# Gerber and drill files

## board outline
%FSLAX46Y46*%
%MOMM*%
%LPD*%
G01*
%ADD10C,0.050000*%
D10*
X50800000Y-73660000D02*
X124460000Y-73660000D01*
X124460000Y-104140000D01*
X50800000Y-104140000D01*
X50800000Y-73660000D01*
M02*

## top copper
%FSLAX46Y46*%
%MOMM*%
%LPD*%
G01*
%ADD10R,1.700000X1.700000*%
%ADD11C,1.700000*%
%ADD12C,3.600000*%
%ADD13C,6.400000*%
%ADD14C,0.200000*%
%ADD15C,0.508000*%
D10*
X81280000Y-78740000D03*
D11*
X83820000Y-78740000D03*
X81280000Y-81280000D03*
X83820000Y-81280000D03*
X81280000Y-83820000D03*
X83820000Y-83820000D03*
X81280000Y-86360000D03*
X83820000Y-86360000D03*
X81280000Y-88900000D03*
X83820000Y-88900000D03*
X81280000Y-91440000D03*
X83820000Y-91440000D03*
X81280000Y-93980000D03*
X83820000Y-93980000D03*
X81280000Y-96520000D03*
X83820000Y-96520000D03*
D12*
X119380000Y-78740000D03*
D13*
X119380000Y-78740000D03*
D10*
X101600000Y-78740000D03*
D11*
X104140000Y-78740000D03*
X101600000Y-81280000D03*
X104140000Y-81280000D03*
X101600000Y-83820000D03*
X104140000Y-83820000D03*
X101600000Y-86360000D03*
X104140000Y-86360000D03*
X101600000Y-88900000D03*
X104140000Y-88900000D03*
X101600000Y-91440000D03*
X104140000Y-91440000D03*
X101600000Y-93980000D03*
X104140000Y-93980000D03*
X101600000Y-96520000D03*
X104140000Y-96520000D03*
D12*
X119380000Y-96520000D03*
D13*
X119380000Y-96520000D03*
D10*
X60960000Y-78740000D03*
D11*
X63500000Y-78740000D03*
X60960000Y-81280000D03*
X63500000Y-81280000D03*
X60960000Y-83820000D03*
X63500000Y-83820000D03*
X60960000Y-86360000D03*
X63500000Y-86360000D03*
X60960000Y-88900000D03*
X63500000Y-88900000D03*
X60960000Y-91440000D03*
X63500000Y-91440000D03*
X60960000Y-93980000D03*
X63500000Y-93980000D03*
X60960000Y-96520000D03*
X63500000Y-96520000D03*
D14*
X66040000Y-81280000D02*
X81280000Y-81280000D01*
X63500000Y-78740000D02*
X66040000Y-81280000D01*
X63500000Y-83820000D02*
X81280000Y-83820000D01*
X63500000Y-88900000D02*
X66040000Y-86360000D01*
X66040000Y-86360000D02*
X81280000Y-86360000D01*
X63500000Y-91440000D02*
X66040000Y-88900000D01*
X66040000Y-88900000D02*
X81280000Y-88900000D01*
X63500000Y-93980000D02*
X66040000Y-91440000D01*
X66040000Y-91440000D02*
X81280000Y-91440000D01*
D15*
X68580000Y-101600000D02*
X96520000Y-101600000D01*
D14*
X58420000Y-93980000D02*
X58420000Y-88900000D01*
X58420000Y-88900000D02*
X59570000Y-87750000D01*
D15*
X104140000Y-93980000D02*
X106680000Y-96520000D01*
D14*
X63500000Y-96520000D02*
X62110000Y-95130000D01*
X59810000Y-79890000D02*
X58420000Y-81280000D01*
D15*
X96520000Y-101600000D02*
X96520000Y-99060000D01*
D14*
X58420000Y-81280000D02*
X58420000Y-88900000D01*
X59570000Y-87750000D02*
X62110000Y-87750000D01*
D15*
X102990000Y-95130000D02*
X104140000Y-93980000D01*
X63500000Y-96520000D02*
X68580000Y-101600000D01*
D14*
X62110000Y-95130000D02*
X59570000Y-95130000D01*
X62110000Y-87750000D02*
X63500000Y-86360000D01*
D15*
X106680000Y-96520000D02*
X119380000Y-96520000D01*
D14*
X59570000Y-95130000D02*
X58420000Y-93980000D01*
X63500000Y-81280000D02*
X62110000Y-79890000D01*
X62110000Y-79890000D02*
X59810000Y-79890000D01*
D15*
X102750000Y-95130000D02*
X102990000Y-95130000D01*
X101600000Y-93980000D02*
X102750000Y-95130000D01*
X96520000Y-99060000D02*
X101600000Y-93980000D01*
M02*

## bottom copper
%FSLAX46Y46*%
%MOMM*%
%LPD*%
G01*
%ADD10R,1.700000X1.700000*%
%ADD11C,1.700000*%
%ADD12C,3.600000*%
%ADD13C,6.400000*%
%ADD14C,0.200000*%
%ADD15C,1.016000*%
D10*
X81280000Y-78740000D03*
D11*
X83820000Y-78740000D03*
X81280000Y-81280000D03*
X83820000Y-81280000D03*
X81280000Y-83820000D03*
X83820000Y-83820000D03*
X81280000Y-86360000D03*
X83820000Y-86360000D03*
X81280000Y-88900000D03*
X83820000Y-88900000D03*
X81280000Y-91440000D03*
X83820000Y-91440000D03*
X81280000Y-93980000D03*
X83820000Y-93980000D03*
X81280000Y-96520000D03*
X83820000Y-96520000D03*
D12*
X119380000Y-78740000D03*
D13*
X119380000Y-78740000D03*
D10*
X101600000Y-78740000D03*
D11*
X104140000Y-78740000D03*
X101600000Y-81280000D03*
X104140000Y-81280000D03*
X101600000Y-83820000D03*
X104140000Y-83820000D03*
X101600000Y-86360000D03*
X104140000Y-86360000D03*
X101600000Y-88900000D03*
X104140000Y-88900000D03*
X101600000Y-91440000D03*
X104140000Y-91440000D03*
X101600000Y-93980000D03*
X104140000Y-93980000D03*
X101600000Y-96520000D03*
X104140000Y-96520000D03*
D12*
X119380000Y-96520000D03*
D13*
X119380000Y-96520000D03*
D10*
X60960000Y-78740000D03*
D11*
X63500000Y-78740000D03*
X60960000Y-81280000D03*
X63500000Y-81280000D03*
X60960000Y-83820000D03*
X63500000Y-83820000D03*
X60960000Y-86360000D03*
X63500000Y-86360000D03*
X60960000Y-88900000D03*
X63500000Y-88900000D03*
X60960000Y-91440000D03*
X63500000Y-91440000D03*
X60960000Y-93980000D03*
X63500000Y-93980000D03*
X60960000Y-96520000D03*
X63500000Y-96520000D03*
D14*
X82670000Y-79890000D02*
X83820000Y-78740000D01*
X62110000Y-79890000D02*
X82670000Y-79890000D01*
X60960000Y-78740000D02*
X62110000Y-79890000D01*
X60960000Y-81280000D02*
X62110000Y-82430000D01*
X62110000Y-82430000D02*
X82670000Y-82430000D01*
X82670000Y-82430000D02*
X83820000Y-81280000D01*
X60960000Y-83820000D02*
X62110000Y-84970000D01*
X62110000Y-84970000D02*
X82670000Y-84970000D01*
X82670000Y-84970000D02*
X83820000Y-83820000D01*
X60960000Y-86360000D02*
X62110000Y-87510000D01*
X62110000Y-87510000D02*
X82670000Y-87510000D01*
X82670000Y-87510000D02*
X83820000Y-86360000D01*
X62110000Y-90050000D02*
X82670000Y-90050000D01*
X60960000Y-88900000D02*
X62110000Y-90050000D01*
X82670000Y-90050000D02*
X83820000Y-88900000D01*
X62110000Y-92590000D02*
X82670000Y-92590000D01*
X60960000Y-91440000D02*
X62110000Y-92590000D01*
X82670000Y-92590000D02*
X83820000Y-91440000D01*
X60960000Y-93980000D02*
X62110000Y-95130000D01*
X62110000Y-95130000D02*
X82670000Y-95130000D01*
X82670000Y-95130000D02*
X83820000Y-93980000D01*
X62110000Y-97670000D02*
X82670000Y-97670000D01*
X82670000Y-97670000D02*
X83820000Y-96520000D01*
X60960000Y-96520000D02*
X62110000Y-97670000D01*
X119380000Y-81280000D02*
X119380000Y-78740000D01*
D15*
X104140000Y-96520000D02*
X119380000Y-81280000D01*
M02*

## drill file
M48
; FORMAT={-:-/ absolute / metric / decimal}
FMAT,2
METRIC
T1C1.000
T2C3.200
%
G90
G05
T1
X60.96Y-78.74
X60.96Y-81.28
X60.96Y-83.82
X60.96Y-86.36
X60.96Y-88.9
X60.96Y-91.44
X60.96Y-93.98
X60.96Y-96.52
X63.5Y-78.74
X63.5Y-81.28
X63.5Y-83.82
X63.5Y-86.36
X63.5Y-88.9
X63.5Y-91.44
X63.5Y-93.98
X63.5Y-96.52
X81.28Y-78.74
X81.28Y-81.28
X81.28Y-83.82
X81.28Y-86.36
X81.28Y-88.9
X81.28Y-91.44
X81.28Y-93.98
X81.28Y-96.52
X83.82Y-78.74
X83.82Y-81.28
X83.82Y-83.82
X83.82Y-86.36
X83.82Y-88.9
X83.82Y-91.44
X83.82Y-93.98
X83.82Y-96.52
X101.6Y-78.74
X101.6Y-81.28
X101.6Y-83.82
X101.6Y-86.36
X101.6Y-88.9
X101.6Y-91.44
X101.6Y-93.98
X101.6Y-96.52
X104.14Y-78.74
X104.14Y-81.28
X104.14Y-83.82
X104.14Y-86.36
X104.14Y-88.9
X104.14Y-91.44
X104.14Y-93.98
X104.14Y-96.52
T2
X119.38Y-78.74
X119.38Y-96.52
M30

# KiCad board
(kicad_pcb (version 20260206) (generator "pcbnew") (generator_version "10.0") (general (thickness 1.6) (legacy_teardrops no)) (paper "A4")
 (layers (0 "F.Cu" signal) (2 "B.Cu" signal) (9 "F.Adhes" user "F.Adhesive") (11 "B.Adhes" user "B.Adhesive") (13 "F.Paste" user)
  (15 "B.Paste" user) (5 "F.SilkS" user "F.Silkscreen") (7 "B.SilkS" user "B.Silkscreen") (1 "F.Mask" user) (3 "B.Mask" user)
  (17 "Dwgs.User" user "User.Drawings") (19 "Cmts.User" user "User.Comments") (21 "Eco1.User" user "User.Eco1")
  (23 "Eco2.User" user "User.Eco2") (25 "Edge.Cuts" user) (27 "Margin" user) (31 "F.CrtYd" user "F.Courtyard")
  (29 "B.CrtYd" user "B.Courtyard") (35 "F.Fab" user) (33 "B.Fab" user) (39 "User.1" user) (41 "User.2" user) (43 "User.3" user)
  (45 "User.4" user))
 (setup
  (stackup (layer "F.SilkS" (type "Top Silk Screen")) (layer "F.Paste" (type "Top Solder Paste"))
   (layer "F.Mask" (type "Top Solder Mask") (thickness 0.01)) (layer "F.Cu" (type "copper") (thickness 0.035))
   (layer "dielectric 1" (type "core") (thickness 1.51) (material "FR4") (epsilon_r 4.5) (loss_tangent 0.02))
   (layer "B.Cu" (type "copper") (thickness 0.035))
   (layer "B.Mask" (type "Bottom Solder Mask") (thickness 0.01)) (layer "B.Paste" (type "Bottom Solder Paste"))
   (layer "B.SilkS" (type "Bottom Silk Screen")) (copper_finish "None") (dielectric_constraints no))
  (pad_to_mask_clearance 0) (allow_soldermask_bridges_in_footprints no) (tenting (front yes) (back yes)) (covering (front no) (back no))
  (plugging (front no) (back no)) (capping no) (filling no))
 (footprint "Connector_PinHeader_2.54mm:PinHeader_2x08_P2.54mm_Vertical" (layer "F.Cu") (at 81.28 78.74)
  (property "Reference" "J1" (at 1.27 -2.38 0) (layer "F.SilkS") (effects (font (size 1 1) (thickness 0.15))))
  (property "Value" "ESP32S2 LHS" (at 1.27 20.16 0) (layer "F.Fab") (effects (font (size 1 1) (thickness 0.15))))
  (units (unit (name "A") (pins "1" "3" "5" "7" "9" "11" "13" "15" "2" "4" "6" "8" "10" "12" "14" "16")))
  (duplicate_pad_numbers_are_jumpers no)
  (pad "1" thru_hole rect (at 0 0) (size 1.7 1.7) (drill 1) (layers "*.Cu" "*.Mask") (remove_unused_layers no)
   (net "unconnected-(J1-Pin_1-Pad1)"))
  (pad "2" thru_hole circle (at 2.54 0) (size 1.7 1.7) (drill 1) (layers "*.Cu" "*.Mask") (remove_unused_layers no) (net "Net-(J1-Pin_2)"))
  (pad "3" thru_hole circle (at 0 2.54) (size 1.7 1.7) (drill 1) (layers "*.Cu" "*.Mask") (remove_unused_layers no) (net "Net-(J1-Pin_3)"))
  (pad "4" thru_hole circle (at 2.54 2.54) (size 1.7 1.7) (drill 1) (layers "*.Cu" "*.Mask") (remove_unused_layers no)
   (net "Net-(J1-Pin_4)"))
  (pad "5" thru_hole circle (at 0 5.08) (size 1.7 1.7) (drill 1) (layers "*.Cu" "*.Mask") (remove_unused_layers no) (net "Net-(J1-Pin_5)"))
  (pad "6" thru_hole circle (at 2.54 5.08) (size 1.7 1.7) (drill 1) (layers "*.Cu" "*.Mask") (remove_unused_layers no)
   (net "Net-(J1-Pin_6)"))
  (pad "7" thru_hole circle (at 0 7.62) (size 1.7 1.7) (drill 1) (layers "*.Cu" "*.Mask") (remove_unused_layers no) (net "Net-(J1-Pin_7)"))
  (pad "8" thru_hole circle (at 2.54 7.62) (size 1.7 1.7) (drill 1) (layers "*.Cu" "*.Mask") (remove_unused_layers no)
   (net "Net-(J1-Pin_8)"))
  (pad "9" thru_hole circle (at 0 10.16) (size 1.7 1.7) (drill 1) (layers "*.Cu" "*.Mask") (remove_unused_layers no) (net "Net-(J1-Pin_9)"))
  (pad "10" thru_hole circle (at 2.54 10.16) (size 1.7 1.7) (drill 1) (layers "*.Cu" "*.Mask") (remove_unused_layers no)
   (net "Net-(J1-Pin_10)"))
  (pad "11" thru_hole circle (at 0 12.7) (size 1.7 1.7) (drill 1) (layers "*.Cu" "*.Mask") (remove_unused_layers no) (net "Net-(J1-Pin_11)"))
  (pad "12" thru_hole circle (at 2.54 12.7) (size 1.7 1.7) (drill 1) (layers "*.Cu" "*.Mask") (remove_unused_layers no)
   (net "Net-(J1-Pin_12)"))
  (pad "13" thru_hole circle (at 0 15.24) (size 1.7 1.7) (drill 1) (layers "*.Cu" "*.Mask") (remove_unused_layers no)
   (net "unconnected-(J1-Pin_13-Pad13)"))
  (pad "14" thru_hole circle (at 2.54 15.24) (size 1.7 1.7) (drill 1) (layers "*.Cu" "*.Mask") (remove_unused_layers no)
   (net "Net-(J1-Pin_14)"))
  (pad "15" thru_hole circle (at 0 17.78) (size 1.7 1.7) (drill 1) (layers "*.Cu" "*.Mask") (remove_unused_layers no)
   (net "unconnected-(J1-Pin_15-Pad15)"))
  (pad "16" thru_hole circle (at 2.54 17.78) (size 1.7 1.7) (drill 1) (layers "*.Cu" "*.Mask") (remove_unused_layers no)
   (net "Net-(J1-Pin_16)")))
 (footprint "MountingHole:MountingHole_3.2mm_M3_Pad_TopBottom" (layer "F.Cu") (at 119.38 78.74)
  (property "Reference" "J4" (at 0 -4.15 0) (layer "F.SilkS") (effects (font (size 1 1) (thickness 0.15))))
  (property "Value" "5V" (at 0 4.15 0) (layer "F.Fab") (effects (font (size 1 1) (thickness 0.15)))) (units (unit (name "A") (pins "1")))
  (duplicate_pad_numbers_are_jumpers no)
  (pad "1" thru_hole circle (at 0 0) (size 3.6 3.6) (drill 3.2) (layers "*.Cu" "*.Mask") (remove_unused_layers no) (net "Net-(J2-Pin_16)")
   (zone_connect 2))
  (pad "1" connect circle (at 0 0) (size 6.4 6.4) (layers "F.Cu" "F.Mask") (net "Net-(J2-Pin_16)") (zone_connect 2))
  (pad "1" connect circle (at 0 0) (size 6.4 6.4) (layers "B.Cu" "B.Mask") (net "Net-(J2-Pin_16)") (zone_connect 2)))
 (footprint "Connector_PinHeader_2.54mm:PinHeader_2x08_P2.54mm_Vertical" (layer "F.Cu") (at 101.6 78.74)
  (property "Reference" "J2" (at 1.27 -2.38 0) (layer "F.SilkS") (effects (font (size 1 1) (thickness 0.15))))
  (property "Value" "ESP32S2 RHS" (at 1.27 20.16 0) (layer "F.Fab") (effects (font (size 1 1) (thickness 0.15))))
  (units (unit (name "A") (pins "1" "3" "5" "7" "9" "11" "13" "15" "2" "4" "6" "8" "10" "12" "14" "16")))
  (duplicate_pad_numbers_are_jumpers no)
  (pad "1" thru_hole rect (at 0 0) (size 1.7 1.7) (drill 1) (layers "*.Cu" "*.Mask") (remove_unused_layers no)
   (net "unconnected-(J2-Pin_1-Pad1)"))
  (pad "2" thru_hole circle (at 2.54 0) (size 1.7 1.7) (drill 1) (layers "*.Cu" "*.Mask") (remove_unused_layers no)
   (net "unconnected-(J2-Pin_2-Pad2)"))
  (pad "3" thru_hole circle (at 0 2.54) (size 1.7 1.7) (drill 1) (layers "*.Cu" "*.Mask") (remove_unused_layers no)
   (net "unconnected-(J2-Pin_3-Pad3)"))
  (pad "4" thru_hole circle (at 2.54 2.54) (size 1.7 1.7) (drill 1) (layers "*.Cu" "*.Mask") (remove_unused_layers no)
   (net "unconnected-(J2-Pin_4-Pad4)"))
  (pad "5" thru_hole circle (at 0 5.08) (size 1.7 1.7) (drill 1) (layers "*.Cu" "*.Mask") (remove_unused_layers no)
   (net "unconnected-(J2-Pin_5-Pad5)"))
  (pad "6" thru_hole circle (at 2.54 5.08) (size 1.7 1.7) (drill 1) (layers "*.Cu" "*.Mask") (remove_unused_layers no)
   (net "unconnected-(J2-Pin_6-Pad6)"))
  (pad "7" thru_hole circle (at 0 7.62) (size 1.7 1.7) (drill 1) (layers "*.Cu" "*.Mask") (remove_unused_layers no)
   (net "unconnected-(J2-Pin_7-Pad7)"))
  (pad "8" thru_hole circle (at 2.54 7.62) (size 1.7 1.7) (drill 1) (layers "*.Cu" "*.Mask") (remove_unused_layers no)
   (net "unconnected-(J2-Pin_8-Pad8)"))
  (pad "9" thru_hole circle (at 0 10.16) (size 1.7 1.7) (drill 1) (layers "*.Cu" "*.Mask") (remove_unused_layers no)
   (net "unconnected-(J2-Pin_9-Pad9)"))
  (pad "10" thru_hole circle (at 2.54 10.16) (size 1.7 1.7) (drill 1) (layers "*.Cu" "*.Mask") (remove_unused_layers no)
   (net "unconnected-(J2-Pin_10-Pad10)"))
  (pad "11" thru_hole circle (at 0 12.7) (size 1.7 1.7) (drill 1) (layers "*.Cu" "*.Mask") (remove_unused_layers no)
   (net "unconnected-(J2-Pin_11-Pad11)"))
  (pad "12" thru_hole circle (at 2.54 12.7) (size 1.7 1.7) (drill 1) (layers "*.Cu" "*.Mask") (remove_unused_layers no)
   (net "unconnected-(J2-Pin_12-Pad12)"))
  (pad "13" thru_hole circle (at 0 15.24) (size 1.7 1.7) (drill 1) (layers "*.Cu" "*.Mask") (remove_unused_layers no)
   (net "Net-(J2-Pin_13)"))
  (pad "14" thru_hole circle (at 2.54 15.24) (size 1.7 1.7) (drill 1) (layers "*.Cu" "*.Mask") (remove_unused_layers no)
   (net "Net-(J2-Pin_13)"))
  (pad "15" thru_hole circle (at 0 17.78) (size 1.7 1.7) (drill 1) (layers "*.Cu" "*.Mask") (remove_unused_layers no)
   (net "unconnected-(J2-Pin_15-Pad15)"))
  (pad "16" thru_hole circle (at 2.54 17.78) (size 1.7 1.7) (drill 1) (layers "*.Cu" "*.Mask") (remove_unused_layers no)
   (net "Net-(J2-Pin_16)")))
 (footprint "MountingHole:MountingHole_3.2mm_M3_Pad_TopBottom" (layer "F.Cu") (at 119.38 96.52)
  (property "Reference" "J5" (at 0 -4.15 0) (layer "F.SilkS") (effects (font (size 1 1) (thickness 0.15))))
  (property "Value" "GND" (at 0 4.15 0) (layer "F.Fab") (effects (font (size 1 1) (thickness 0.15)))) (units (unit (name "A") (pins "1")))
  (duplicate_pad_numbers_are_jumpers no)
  (pad "1" thru_hole circle (at 0 0) (size 3.6 3.6) (drill 3.2) (layers "*.Cu" "*.Mask") (remove_unused_layers no) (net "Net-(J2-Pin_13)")
   (zone_connect 2))
  (pad "1" connect circle (at 0 0) (size 6.4 6.4) (layers "F.Cu" "F.Mask") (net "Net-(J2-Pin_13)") (zone_connect 2))
  (pad "1" connect circle (at 0 0) (size 6.4 6.4) (layers "B.Cu" "B.Mask") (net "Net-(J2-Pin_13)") (zone_connect 2)))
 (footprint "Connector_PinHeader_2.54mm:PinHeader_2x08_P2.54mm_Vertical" (layer "F.Cu") (at 60.96 78.74)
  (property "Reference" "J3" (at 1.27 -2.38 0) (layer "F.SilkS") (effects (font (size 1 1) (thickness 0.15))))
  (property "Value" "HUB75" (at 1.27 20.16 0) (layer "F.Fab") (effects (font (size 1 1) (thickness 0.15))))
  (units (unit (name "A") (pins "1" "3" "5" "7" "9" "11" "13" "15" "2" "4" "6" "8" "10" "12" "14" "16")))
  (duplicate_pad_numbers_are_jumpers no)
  (pad "1" thru_hole rect (at 0 0) (size 1.7 1.7) (drill 1) (layers "*.Cu" "*.Mask") (remove_unused_layers no) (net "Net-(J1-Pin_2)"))
  (pad "2" thru_hole circle (at 2.54 0) (size 1.7 1.7) (drill 1) (layers "*.Cu" "*.Mask") (remove_unused_layers no) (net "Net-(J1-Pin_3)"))
  (pad "3" thru_hole circle (at 0 2.54) (size 1.7 1.7) (drill 1) (layers "*.Cu" "*.Mask") (remove_unused_layers no) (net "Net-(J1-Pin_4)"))
  (pad "4" thru_hole circle (at 2.54 2.54) (size 1.7 1.7) (drill 1) (layers "*.Cu" "*.Mask") (remove_unused_layers no)
   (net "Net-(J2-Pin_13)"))
  (pad "5" thru_hole circle (at 0 5.08) (size 1.7 1.7) (drill 1) (layers "*.Cu" "*.Mask") (remove_unused_layers no) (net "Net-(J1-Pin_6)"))
  (pad "6" thru_hole circle (at 2.54 5.08) (size 1.7 1.7) (drill 1) (layers "*.Cu" "*.Mask") (remove_unused_layers no)
   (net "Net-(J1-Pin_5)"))
  (pad "7" thru_hole circle (at 0 7.62) (size 1.7 1.7) (drill 1) (layers "*.Cu" "*.Mask") (remove_unused_layers no) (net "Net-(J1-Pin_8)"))
  (pad "8" thru_hole circle (at 2.54 7.62) (size 1.7 1.7) (drill 1) (layers "*.Cu" "*.Mask") (remove_unused_layers no)
   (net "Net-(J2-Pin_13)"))
  (pad "9" thru_hole circle (at 0 10.16) (size 1.7 1.7) (drill 1) (layers "*.Cu" "*.Mask") (remove_unused_layers no) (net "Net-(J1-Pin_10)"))
  (pad "10" thru_hole circle (at 2.54 10.16) (size 1.7 1.7) (drill 1) (layers "*.Cu" "*.Mask") (remove_unused_layers no)
   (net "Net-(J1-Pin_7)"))
  (pad "11" thru_hole circle (at 0 12.7) (size 1.7 1.7) (drill 1) (layers "*.Cu" "*.Mask") (remove_unused_layers no) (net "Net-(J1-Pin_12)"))
  (pad "12" thru_hole circle (at 2.54 12.7) (size 1.7 1.7) (drill 1) (layers "*.Cu" "*.Mask") (remove_unused_layers no)
   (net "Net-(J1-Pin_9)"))
  (pad "13" thru_hole circle (at 0 15.24) (size 1.7 1.7) (drill 1) (layers "*.Cu" "*.Mask") (remove_unused_layers no)
   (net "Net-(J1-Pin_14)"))
  (pad "14" thru_hole circle (at 2.54 15.24) (size 1.7 1.7) (drill 1) (layers "*.Cu" "*.Mask") (remove_unused_layers no)
   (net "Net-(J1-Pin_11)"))
  (pad "15" thru_hole circle (at 0 17.78) (size 1.7 1.7) (drill 1) (layers "*.Cu" "*.Mask") (remove_unused_layers no)
   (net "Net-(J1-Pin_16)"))
  (pad "16" thru_hole circle (at 2.54 17.78) (size 1.7 1.7) (drill 1) (layers "*.Cu" "*.Mask") (remove_unused_layers no)
   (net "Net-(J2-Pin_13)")))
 (gr_rect (start 50.8 73.66) (end 124.46 104.14) (stroke (width 0.05) (type default)) (fill no) (layer "Edge.Cuts"))
 (segment (start 82.67 79.89) (end 83.82 78.74) (width 0.2) (layer "B.Cu") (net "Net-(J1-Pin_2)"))
 (segment (start 62.11 79.89) (end 82.67 79.89) (width 0.2) (layer "B.Cu") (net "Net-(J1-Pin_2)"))
 (segment (start 60.96 78.74) (end 62.11 79.89) (width 0.2) (layer "B.Cu") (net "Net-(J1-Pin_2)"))
 (segment (start 66.04 81.28) (end 81.28 81.28) (width 0.2) (layer "F.Cu") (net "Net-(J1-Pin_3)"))
 (segment (start 63.5 78.74) (end 66.04 81.28) (width 0.2) (layer "F.Cu") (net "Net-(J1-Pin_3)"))
 (segment (start 60.96 81.28) (end 62.11 82.43) (width 0.2) (layer "B.Cu") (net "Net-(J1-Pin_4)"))
 (segment (start 62.11 82.43) (end 82.67 82.43) (width 0.2) (layer "B.Cu") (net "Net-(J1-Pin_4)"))
 (segment (start 82.67 82.43) (end 83.82 81.28) (width 0.2) (layer "B.Cu") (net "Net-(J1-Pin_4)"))
 (segment (start 63.5 83.82) (end 81.28 83.82) (width 0.2) (layer "F.Cu") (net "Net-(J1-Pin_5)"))
 (segment (start 60.96 83.82) (end 62.11 84.97) (width 0.2) (layer "B.Cu") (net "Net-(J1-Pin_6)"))
 (segment (start 62.11 84.97) (end 82.67 84.97) (width 0.2) (layer "B.Cu") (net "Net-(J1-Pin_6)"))
 (segment (start 82.67 84.97) (end 83.82 83.82) (width 0.2) (layer "B.Cu") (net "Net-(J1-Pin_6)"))
 (segment (start 63.5 88.9) (end 66.04 86.36) (width 0.2) (layer "F.Cu") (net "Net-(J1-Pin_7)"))
 (segment (start 66.04 86.36) (end 81.28 86.36) (width 0.2) (layer "F.Cu") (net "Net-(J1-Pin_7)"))
 (segment (start 60.96 86.36) (end 62.11 87.51) (width 0.2) (layer "B.Cu") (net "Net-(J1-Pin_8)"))
 (segment (start 62.11 87.51) (end 82.67 87.51) (width 0.2) (layer "B.Cu") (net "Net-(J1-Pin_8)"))
 (segment (start 82.67 87.51) (end 83.82 86.36) (width 0.2) (layer "B.Cu") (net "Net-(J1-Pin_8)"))
 (segment (start 63.5 91.44) (end 66.04 88.9) (width 0.2) (layer "F.Cu") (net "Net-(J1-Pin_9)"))
 (segment (start 66.04 88.9) (end 81.28 88.9) (width 0.2) (layer "F.Cu") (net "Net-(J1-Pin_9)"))
 (segment (start 62.11 90.05) (end 82.67 90.05) (width 0.2) (layer "B.Cu") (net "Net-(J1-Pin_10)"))
 (segment (start 60.96 88.9) (end 62.11 90.05) (width 0.2) (layer "B.Cu") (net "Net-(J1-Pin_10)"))
 (segment (start 82.67 90.05) (end 83.82 88.9) (width 0.2) (layer "B.Cu") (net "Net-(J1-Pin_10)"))
 (segment (start 63.5 93.98) (end 66.04 91.44) (width 0.2) (layer "F.Cu") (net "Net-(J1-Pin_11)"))
 (segment (start 66.04 91.44) (end 81.28 91.44) (width 0.2) (layer "F.Cu") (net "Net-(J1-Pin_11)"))
 (segment (start 62.11 92.59) (end 82.67 92.59) (width 0.2) (layer "B.Cu") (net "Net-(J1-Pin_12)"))
 (segment (start 60.96 91.44) (end 62.11 92.59) (width 0.2) (layer "B.Cu") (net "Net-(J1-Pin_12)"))
 (segment (start 82.67 92.59) (end 83.82 91.44) (width 0.2) (layer "B.Cu") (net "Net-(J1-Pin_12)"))
 (segment (start 60.96 93.98) (end 62.11 95.13) (width 0.2) (layer "B.Cu") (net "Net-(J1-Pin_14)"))
 (segment (start 62.11 95.13) (end 82.67 95.13) (width 0.2) (layer "B.Cu") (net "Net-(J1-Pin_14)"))
 (segment (start 82.67 95.13) (end 83.82 93.98) (width 0.2) (layer "B.Cu") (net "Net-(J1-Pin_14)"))
 (segment (start 62.11 97.67) (end 82.67 97.67) (width 0.2) (layer "B.Cu") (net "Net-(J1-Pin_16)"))
 (segment (start 82.67 97.67) (end 83.82 96.52) (width 0.2) (layer "B.Cu") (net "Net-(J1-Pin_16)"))
 (segment (start 60.96 96.52) (end 62.11 97.67) (width 0.2) (layer "B.Cu") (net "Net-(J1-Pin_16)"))
 (segment (start 119.38 81.28) (end 119.38 78.74) (width 0.2) (layer "B.Cu") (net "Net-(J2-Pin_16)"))
 (segment (start 104.14 96.52) (end 119.38 81.28) (width 1.016) (layer "B.Cu") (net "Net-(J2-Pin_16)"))
 (segment (start 68.58 101.6) (end 96.52 101.6) (width 0.508) (layer "F.Cu") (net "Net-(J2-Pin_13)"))
 (segment (start 58.42 93.98) (end 58.42 88.9) (width 0.2) (layer "F.Cu") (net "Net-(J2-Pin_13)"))
 (segment (start 58.42 88.9) (end 59.57 87.75) (width 0.2) (layer "F.Cu") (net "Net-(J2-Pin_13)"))
 (segment (start 104.14 93.98) (end 106.68 96.52) (width 0.508) (layer "F.Cu") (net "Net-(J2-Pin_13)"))
 (segment (start 63.5 96.52) (end 62.11 95.13) (width 0.2) (layer "F.Cu") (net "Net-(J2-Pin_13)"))
 (segment (start 59.81 79.89) (end 58.42 81.28) (width 0.2) (layer "F.Cu") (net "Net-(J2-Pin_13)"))
 (segment (start 96.52 101.6) (end 96.52 99.06) (width 0.508) (layer "F.Cu") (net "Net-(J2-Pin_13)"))
 (segment (start 58.42 81.28) (end 58.42 88.9) (width 0.2) (layer "F.Cu") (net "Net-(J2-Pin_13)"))
 (segment (start 59.57 87.75) (end 62.11 87.75) (width 0.2) (layer "F.Cu") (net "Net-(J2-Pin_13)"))
 (segment (start 102.99 95.13) (end 104.14 93.98) (width 0.508) (layer "F.Cu") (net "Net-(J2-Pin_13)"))
 (segment (start 63.5 96.52) (end 68.58 101.6) (width 0.508) (layer "F.Cu") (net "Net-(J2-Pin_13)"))
 (segment (start 62.11 95.13) (end 59.57 95.13) (width 0.2) (layer "F.Cu") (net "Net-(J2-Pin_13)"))
 (segment (start 62.11 87.75) (end 63.5 86.36) (width 0.2) (layer "F.Cu") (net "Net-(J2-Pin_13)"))
 (segment (start 106.68 96.52) (end 119.38 96.52) (width 0.508) (layer "F.Cu") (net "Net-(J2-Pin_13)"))
 (segment (start 59.57 95.13) (end 58.42 93.98) (width 0.2) (layer "F.Cu") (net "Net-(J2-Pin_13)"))
 (segment (start 63.5 81.28) (end 62.11 79.89) (width 0.2) (layer "F.Cu") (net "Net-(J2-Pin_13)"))
 (segment (start 62.11 79.89) (end 59.81 79.89) (width 0.2) (layer "F.Cu") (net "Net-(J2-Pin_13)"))
 (segment (start 102.75 95.13) (end 102.99 95.13) (width 0.508) (layer "F.Cu") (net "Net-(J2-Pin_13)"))
 (segment (start 101.6 93.98) (end 102.75 95.13) (width 0.508) (layer "F.Cu") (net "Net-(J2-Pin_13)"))
 (segment (start 96.52 99.06) (end 101.6 93.98) (width 0.508) (layer "F.Cu") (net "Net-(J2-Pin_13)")))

